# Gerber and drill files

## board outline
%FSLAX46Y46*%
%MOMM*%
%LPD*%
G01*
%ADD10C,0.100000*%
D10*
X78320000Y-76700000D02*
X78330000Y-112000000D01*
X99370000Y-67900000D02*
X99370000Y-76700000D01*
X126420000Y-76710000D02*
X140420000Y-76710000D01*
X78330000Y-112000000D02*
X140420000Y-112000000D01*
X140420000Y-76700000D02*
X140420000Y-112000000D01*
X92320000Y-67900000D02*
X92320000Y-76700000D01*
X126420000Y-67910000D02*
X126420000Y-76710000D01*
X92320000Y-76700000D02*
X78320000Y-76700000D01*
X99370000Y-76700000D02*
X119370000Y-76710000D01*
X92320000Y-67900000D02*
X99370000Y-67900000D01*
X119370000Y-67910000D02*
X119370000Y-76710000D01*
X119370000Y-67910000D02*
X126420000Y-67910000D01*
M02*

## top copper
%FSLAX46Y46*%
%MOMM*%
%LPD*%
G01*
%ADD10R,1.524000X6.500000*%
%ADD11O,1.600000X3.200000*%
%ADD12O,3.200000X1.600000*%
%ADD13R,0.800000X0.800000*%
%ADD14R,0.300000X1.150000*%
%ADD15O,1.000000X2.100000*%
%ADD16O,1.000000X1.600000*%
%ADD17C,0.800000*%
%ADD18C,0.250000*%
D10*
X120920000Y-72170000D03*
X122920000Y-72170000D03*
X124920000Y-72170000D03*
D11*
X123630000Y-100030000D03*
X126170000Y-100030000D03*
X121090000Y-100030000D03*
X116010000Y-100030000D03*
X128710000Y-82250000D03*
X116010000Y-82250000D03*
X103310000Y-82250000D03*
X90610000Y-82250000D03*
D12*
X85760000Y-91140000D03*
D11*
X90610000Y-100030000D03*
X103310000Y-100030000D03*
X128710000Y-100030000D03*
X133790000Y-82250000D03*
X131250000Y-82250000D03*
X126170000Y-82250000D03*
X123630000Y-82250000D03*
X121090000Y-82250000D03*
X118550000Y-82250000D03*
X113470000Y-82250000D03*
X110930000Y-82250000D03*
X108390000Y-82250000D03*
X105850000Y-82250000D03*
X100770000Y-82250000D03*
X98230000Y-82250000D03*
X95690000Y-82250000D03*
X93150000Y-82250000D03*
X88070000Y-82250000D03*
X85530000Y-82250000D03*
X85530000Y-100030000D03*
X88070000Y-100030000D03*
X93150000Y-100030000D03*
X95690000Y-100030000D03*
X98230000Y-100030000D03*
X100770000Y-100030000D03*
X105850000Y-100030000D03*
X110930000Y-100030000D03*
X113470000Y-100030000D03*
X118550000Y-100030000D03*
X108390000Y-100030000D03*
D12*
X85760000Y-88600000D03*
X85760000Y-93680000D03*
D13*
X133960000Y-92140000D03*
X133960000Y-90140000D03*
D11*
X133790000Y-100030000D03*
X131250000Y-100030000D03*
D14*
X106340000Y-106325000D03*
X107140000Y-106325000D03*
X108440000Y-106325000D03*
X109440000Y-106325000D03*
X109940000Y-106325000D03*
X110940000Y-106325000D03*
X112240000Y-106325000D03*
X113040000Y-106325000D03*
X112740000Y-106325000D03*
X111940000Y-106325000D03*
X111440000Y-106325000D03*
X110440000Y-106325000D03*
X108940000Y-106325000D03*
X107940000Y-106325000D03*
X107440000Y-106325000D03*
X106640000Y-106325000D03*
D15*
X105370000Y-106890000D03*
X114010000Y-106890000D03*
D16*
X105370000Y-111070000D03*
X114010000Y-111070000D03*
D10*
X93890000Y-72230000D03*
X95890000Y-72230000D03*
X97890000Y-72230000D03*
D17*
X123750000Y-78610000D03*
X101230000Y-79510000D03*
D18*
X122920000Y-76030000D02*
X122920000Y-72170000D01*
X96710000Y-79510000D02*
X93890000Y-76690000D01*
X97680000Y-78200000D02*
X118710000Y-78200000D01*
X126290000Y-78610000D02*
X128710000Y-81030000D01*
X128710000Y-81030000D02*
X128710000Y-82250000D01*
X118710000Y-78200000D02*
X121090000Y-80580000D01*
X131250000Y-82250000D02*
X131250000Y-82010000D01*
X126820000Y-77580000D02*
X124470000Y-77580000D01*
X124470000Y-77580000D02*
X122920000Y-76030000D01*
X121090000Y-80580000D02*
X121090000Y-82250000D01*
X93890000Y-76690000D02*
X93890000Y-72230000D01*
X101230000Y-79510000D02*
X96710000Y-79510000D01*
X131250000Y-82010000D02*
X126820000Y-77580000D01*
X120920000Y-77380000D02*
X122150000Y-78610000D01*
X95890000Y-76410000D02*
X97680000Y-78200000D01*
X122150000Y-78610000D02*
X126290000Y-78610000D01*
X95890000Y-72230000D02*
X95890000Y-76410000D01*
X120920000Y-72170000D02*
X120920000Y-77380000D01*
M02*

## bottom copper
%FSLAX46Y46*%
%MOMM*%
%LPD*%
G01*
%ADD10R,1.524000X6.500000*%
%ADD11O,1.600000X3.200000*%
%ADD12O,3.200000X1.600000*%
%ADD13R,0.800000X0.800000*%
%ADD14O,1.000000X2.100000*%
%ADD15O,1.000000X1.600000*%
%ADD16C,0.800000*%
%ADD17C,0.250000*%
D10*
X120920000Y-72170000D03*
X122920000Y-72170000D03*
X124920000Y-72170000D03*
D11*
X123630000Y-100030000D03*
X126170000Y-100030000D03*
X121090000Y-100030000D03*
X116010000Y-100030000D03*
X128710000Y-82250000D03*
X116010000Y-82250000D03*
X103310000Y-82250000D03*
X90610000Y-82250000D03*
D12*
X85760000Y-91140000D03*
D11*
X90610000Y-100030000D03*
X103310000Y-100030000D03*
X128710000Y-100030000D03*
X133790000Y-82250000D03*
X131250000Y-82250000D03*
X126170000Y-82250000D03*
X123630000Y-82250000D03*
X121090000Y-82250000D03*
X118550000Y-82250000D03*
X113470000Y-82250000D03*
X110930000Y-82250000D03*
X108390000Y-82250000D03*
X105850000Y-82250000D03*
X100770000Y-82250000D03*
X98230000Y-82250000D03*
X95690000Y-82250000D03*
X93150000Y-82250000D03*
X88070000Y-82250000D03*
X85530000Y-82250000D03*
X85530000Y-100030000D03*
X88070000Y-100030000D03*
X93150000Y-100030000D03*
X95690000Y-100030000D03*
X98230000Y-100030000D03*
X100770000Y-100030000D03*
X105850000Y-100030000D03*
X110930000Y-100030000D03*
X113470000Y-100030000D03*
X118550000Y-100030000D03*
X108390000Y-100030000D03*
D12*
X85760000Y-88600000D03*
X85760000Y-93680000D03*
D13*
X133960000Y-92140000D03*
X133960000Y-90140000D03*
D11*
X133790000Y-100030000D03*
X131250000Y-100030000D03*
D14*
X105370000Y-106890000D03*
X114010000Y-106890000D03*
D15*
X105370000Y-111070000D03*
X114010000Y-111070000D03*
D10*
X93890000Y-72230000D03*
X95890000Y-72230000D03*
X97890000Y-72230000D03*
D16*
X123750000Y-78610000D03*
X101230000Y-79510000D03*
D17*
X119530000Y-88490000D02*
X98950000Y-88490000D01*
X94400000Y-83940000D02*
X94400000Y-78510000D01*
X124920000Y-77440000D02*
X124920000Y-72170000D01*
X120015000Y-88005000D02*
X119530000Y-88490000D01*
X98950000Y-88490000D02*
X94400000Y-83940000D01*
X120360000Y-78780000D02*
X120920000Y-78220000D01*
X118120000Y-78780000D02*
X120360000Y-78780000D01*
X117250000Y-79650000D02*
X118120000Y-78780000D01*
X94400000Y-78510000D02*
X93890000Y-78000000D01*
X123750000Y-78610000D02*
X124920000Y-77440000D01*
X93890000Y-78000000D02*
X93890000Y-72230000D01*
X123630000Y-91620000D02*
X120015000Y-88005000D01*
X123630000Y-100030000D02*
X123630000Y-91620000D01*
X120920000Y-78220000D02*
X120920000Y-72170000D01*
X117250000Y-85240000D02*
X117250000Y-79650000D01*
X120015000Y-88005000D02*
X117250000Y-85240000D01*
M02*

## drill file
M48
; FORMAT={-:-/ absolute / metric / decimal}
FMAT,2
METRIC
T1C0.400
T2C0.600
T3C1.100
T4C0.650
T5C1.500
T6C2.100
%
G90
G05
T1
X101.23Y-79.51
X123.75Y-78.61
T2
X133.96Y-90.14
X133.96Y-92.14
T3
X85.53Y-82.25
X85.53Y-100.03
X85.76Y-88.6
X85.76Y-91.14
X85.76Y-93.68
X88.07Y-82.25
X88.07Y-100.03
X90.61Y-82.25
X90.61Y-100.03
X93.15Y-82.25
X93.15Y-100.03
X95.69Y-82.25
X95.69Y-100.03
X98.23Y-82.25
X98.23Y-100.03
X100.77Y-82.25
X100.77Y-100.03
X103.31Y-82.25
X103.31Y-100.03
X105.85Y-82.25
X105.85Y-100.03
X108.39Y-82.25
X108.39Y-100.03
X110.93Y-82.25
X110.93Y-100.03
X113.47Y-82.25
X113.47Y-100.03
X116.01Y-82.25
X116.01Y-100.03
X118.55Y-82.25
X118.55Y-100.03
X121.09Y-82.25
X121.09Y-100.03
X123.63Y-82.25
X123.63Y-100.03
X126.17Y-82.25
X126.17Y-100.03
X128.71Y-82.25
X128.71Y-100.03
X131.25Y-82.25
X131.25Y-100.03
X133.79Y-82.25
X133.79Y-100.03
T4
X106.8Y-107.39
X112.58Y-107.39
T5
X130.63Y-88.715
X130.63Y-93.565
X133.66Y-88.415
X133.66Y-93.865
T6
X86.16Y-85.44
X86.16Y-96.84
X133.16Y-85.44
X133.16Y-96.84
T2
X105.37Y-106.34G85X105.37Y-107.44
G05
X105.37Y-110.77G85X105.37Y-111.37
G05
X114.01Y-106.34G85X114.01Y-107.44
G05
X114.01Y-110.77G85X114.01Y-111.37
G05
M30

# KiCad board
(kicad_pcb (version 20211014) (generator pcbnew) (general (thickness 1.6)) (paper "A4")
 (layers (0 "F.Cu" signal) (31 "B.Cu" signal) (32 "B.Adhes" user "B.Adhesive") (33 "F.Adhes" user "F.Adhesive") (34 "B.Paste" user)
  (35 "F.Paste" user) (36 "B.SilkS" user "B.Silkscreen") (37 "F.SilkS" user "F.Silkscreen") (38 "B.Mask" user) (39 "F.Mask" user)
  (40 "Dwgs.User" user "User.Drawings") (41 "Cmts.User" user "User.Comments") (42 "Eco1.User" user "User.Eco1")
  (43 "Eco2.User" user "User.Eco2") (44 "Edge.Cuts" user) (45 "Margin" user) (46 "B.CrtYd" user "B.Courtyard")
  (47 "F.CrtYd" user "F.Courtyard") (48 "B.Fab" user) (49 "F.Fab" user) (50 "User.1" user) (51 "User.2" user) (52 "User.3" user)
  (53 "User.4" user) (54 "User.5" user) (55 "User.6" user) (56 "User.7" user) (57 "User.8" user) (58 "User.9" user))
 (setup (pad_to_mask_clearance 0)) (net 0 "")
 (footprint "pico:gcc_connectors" (layer "F.Cu") (at 123.27 72.17)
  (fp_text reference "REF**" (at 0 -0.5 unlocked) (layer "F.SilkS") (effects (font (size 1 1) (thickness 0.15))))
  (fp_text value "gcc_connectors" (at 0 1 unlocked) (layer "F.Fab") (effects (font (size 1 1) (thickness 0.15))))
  (pad "1" smd rect (at -2.35 0) (size 1.524 6.5) (layers "F.Cu" "F.Paste" "F.Mask"))
  (pad "2" smd rect (at -0.35 0) (size 1.524 6.5) (layers "F.Cu" "F.Paste" "F.Mask"))
  (pad "3" smd rect (at 1.65 0) (size 1.524 6.5) (layers "F.Cu" "F.Paste" "F.Mask"))
  (pad "4" smd rect (at -2.35 0) (size 1.524 6.5) (layers "B.Cu" "B.Paste" "B.Mask"))
  (pad "5" smd rect (at -0.35 0) (size 1.524 6.5) (layers "B.Cu" "B.Paste" "B.Mask"))
  (pad "6" smd rect (at 1.65 0) (size 1.524 6.5) (layers "B.Cu" "B.Paste" "B.Mask")))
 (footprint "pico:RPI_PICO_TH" (layer "F.Cu") (at 109.66 91.14 -90)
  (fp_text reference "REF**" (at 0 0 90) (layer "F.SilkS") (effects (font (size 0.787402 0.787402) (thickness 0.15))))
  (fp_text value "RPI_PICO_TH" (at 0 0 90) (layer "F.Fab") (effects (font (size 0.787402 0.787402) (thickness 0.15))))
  (pad "" np_thru_hole circle locked (at -5.7 23.5 270) (size 2.1 2.1) (drill 2.1) (layers *.Cu *.Mask))
  (pad "" np_thru_hole circle locked (at -2.425 -20.97 270) (size 1.5 1.5) (drill 1.5) (layers *.Cu *.Mask))
  (pad "" np_thru_hole circle locked (at -5.7 -23.5 270) (size 2.1 2.1) (drill 2.1) (layers *.Cu *.Mask))
  (pad "" np_thru_hole circle locked (at 2.425 -20.97 270) (size 1.5 1.5) (drill 1.5) (layers *.Cu *.Mask))
  (pad "" np_thru_hole circle locked (at 2.725 -24 270) (size 1.5 1.5) (drill 1.5) (layers *.Cu *.Mask))
  (pad "" np_thru_hole circle locked (at 5.7 23.5 270) (size 2.1 2.1) (drill 2.1) (layers *.Cu *.Mask))
  (pad "" np_thru_hole circle locked (at 5.7 -23.5 270) (size 2.1 2.1) (drill 2.1) (layers *.Cu *.Mask))
  (pad "" np_thru_hole circle locked (at -2.725 -24 270) (size 1.5 1.5) (drill 1.5) (layers *.Cu *.Mask))
  (pad "3V3" thru_hole oval locked (at 8.89 -13.97 270) (size 3.2 1.6) (drill 1.1) (layers *.Cu *.Mask))
  (pad "3V3_EN" thru_hole oval locked (at 8.89 -16.51 270) (size 3.2 1.6) (drill 1.1) (layers *.Cu *.Mask))
  (pad "ADC_VREF" thru_hole oval locked (at 8.89 -11.43 270) (size 3.2 1.6) (drill 1.1) (layers *.Cu *.Mask))
  (pad "AGND" thru_hole oval locked (at 8.89 -6.35 270) (size 3.2 1.6) (drill 1.1) (layers *.Cu *.Mask))
  (pad "GND@1" thru_hole oval locked (at -8.89 -19.05 270) (size 3.2 1.6) (drill 1.1) (layers *.Cu *.Mask))
  (pad "GND@2" thru_hole oval locked (at -8.89 -6.35 270) (size 3.2 1.6) (drill 1.1) (layers *.Cu *.Mask))
  (pad "GND@3" thru_hole oval locked (at -8.89 6.35 270) (size 3.2 1.6) (drill 1.1) (layers *.Cu *.Mask))
  (pad "GND@4" thru_hole oval locked (at -8.89 19.05 270) (size 3.2 1.6) (drill 1.1) (layers *.Cu *.Mask))
  (pad "GND@5" thru_hole oval locked (at 0 23.9 270) (size 1.6 3.2) (drill 1.1) (layers *.Cu *.Mask))
  (pad "GND@6" thru_hole oval locked (at 8.89 19.05 270) (size 3.2 1.6) (drill 1.1) (layers *.Cu *.Mask))
  (pad "GND@7" thru_hole oval locked (at 8.89 6.35 270) (size 3.2 1.6) (drill 1.1) (layers *.Cu *.Mask))
  (pad "GND@8" thru_hole oval locked (at 8.89 -19.05 270) (size 3.2 1.6) (drill 1.1) (layers *.Cu *.Mask))
  (pad "GP0" thru_hole oval locked (at -8.89 -24.13 270) (size 3.2 1.6) (drill 1.1) (layers *.Cu *.Mask))
  (pad "GP1" thru_hole oval locked (at -8.89 -21.59 270) (size 3.2 1.6) (drill 1.1) (layers *.Cu *.Mask))
  (pad "GP2" thru_hole oval locked (at -8.89 -16.51 270) (size 3.2 1.6) (drill 1.1) (layers *.Cu *.Mask))
  (pad "GP3" thru_hole oval locked (at -8.89 -13.97 270) (size 3.2 1.6) (drill 1.1) (layers *.Cu *.Mask))
  (pad "GP4" thru_hole oval locked (at -8.89 -11.43 270) (size 3.2 1.6) (drill 1.1) (layers *.Cu *.Mask))
  (pad "GP5" thru_hole oval locked (at -8.89 -8.89 270) (size 3.2 1.6) (drill 1.1) (layers *.Cu *.Mask))
  (pad "GP6" thru_hole oval locked (at -8.89 -3.81 270) (size 3.2 1.6) (drill 1.1) (layers *.Cu *.Mask))
  (pad "GP7" thru_hole oval locked (at -8.89 -1.27 270) (size 3.2 1.6) (drill 1.1) (layers *.Cu *.Mask))
  (pad "GP8" thru_hole oval locked (at -8.89 1.27 270) (size 3.2 1.6) (drill 1.1) (layers *.Cu *.Mask))
  (pad "GP9" thru_hole oval locked (at -8.89 3.81 270) (size 3.2 1.6) (drill 1.1) (layers *.Cu *.Mask))
  (pad "GP10" thru_hole oval locked (at -8.89 8.89 270) (size 3.2 1.6) (drill 1.1) (layers *.Cu *.Mask))
  (pad "GP11" thru_hole oval locked (at -8.89 11.43 270) (size 3.2 1.6) (drill 1.1) (layers *.Cu *.Mask))
  (pad "GP12" thru_hole oval locked (at -8.89 13.97 270) (size 3.2 1.6) (drill 1.1) (layers *.Cu *.Mask))
  (pad "GP13" thru_hole oval locked (at -8.89 16.51 270) (size 3.2 1.6) (drill 1.1) (layers *.Cu *.Mask))
  (pad "GP14" thru_hole oval locked (at -8.89 21.59 270) (size 3.2 1.6) (drill 1.1) (layers *.Cu *.Mask))
  (pad "GP15" thru_hole oval locked (at -8.89 24.13 270) (size 3.2 1.6) (drill 1.1) (layers *.Cu *.Mask))
  (pad "GP16" thru_hole oval locked (at 8.89 24.13 270) (size 3.2 1.6) (drill 1.1) (layers *.Cu *.Mask))
  (pad "GP17" thru_hole oval locked (at 8.89 21.59 270) (size 3.2 1.6) (drill 1.1) (layers *.Cu *.Mask))
  (pad "GP18" thru_hole oval locked (at 8.89 16.51 270) (size 3.2 1.6) (drill 1.1) (layers *.Cu *.Mask))
  (pad "GP19" thru_hole oval locked (at 8.89 13.97 270) (size 3.2 1.6) (drill 1.1) (layers *.Cu *.Mask))
  (pad "GP20" thru_hole oval locked (at 8.89 11.43 270) (size 3.2 1.6) (drill 1.1) (layers *.Cu *.Mask))
  (pad "GP21" thru_hole oval locked (at 8.89 8.89 270) (size 3.2 1.6) (drill 1.1) (layers *.Cu *.Mask))
  (pad "GP22" thru_hole oval locked (at 8.89 3.81 270) (size 3.2 1.6) (drill 1.1) (layers *.Cu *.Mask))
  (pad "GP26_A0" thru_hole oval locked (at 8.89 -1.27 270) (size 3.2 1.6) (drill 1.1) (layers *.Cu *.Mask))
  (pad "GP27_A1" thru_hole oval locked (at 8.89 -3.81 270) (size 3.2 1.6) (drill 1.1) (layers *.Cu *.Mask))
  (pad "GP28_A2" thru_hole oval locked (at 8.89 -8.89 270) (size 3.2 1.6) (drill 1.1) (layers *.Cu *.Mask))
  (pad "RUN" thru_hole oval locked (at 8.89 1.27 270) (size 3.2 1.6) (drill 1.1) (layers *.Cu *.Mask))
  (pad "SWCLK" thru_hole oval locked (at -2.54 23.9 270) (size 1.6 3.2) (drill 1.1) (layers *.Cu *.Mask))
  (pad "SWDIO" thru_hole oval locked (at 2.54 23.9 270) (size 1.6 3.2) (drill 1.1) (layers *.Cu *.Mask))
  (pad "TP2" thru_hole rect locked (at 1 -24.3 270) (size 0.8 0.8) (drill 0.6) (layers *.Cu *.Mask))
  (pad "TP3" thru_hole rect locked (at -1 -24.3 270) (size 0.8 0.8) (drill 0.6) (layers *.Cu *.Mask))
  (pad "VBUS" thru_hole oval locked (at 8.89 -24.13 270) (size 3.2 1.6) (drill 1.1) (layers *.Cu *.Mask))
  (pad "VSYS" thru_hole oval locked (at 8.89 -21.59 270) (size 3.2 1.6) (drill 1.1) (layers *.Cu *.Mask)))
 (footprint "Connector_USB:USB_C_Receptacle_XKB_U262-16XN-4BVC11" (layer "F.Cu") (at 109.69 109.995)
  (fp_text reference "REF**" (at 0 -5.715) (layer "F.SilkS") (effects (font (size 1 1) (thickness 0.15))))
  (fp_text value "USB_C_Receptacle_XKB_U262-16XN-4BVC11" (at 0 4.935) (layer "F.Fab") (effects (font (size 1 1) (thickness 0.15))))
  (pad "" np_thru_hole circle (at -2.89 -2.605) (size 0.65 0.65) (drill 0.65) (layers *.Cu *.Mask))
  (pad "" np_thru_hole circle (at 2.89 -2.605) (size 0.65 0.65) (drill 0.65) (layers *.Cu *.Mask))
  (pad "A1" smd rect (at -3.35 -3.67) (size 0.3 1.15) (layers "F.Cu" "F.Paste" "F.Mask"))
  (pad "A4" smd rect (at -2.55 -3.67) (size 0.3 1.15) (layers "F.Cu" "F.Paste" "F.Mask"))
  (pad "A5" smd rect (at -1.25 -3.67) (size 0.3 1.15) (layers "F.Cu" "F.Paste" "F.Mask"))
  (pad "A6" smd rect (at -0.25 -3.67) (size 0.3 1.15) (layers "F.Cu" "F.Paste" "F.Mask"))
  (pad "A7" smd rect (at 0.25 -3.67) (size 0.3 1.15) (layers "F.Cu" "F.Paste" "F.Mask"))
  (pad "A8" smd rect (at 1.25 -3.67) (size 0.3 1.15) (layers "F.Cu" "F.Paste" "F.Mask"))
  (pad "A9" smd rect (at 2.55 -3.67) (size 0.3 1.15) (layers "F.Cu" "F.Paste" "F.Mask"))
  (pad "A12" smd rect (at 3.35 -3.67) (size 0.3 1.15) (layers "F.Cu" "F.Paste" "F.Mask"))
  (pad "B1" smd rect (at 3.05 -3.67) (size 0.3 1.15) (layers "F.Cu" "F.Paste" "F.Mask"))
  (pad "B4" smd rect (at 2.25 -3.67) (size 0.3 1.15) (layers "F.Cu" "F.Paste" "F.Mask"))
  (pad "B5" smd rect (at 1.75 -3.67) (size 0.3 1.15) (layers "F.Cu" "F.Paste" "F.Mask"))
  (pad "B6" smd rect (at 0.75 -3.67) (size 0.3 1.15) (layers "F.Cu" "F.Paste" "F.Mask"))
  (pad "B7" smd rect (at -0.75 -3.67) (size 0.3 1.15) (layers "F.Cu" "F.Paste" "F.Mask"))
  (pad "B8" smd rect (at -1.75 -3.67) (size 0.3 1.15) (layers "F.Cu" "F.Paste" "F.Mask"))
  (pad "B9" smd rect (at -2.25 -3.67) (size 0.3 1.15) (layers "F.Cu" "F.Paste" "F.Mask"))
  (pad "B12" smd rect (at -3.05 -3.67) (size 0.3 1.15) (layers "F.Cu" "F.Paste" "F.Mask"))
  (pad "S1" thru_hole oval (at -4.32 -3.105) (size 1 2.1) (drill oval 0.6 1.7) (layers *.Cu *.Mask))
  (pad "S1" thru_hole oval (at 4.32 -3.105) (size 1 2.1) (drill oval 0.6 1.7) (layers *.Cu *.Mask))
  (pad "S1" thru_hole oval (at -4.32 1.075) (size 1 1.6) (drill oval 0.6 1.2) (layers *.Cu *.Mask))
  (pad "S1" thru_hole oval (at 4.32 1.075) (size 1 1.6) (drill oval 0.6 1.2) (layers *.Cu *.Mask)))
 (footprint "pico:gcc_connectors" (layer "F.Cu") (at 96.24 72.23)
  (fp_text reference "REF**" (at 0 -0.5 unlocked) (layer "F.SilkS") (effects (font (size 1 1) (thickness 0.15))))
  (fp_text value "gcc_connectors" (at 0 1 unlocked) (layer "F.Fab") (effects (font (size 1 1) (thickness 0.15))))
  (pad "1" smd rect (at -2.35 0) (size 1.524 6.5) (layers "F.Cu" "F.Paste" "F.Mask"))
  (pad "2" smd rect (at -0.35 0) (size 1.524 6.5) (layers "F.Cu" "F.Paste" "F.Mask"))
  (pad "3" smd rect (at 1.65 0) (size 1.524 6.5) (layers "F.Cu" "F.Paste" "F.Mask"))
  (pad "4" smd rect (at -2.35 0) (size 1.524 6.5) (layers "B.Cu" "B.Paste" "B.Mask"))
  (pad "5" smd rect (at -0.35 0) (size 1.524 6.5) (layers "B.Cu" "B.Paste" "B.Mask"))
  (pad "6" smd rect (at 1.65 0) (size 1.524 6.5) (layers "B.Cu" "B.Paste" "B.Mask")))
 (gr_line (start 78.32 76.7) (end 78.33 112) (layer "Edge.Cuts") (width 0.1))
 (gr_line (start 99.37 67.9) (end 99.37 76.7) (layer "Edge.Cuts") (width 0.1))
 (gr_line (start 126.42 76.71) (end 140.42 76.71) (layer "Edge.Cuts") (width 0.1))
 (gr_line (start 78.33 112) (end 140.42 112) (layer "Edge.Cuts") (width 0.1))
 (gr_line (start 140.42 76.7) (end 140.42 112) (layer "Edge.Cuts") (width 0.1))
 (gr_line (start 92.32 67.9) (end 92.32 76.7) (layer "Edge.Cuts") (width 0.1))
 (gr_line (start 126.42 67.91) (end 126.42 76.71) (layer "Edge.Cuts") (width 0.1))
 (gr_line (start 92.32 76.7) (end 78.32 76.7) (layer "Edge.Cuts") (width 0.1))
 (gr_line (start 99.37 76.7) (end 119.37 76.71) (layer "Edge.Cuts") (width 0.1))
 (gr_line (start 92.32 67.9) (end 99.37 67.9) (layer "Edge.Cuts") (width 0.1))
 (gr_line (start 119.37 67.91) (end 119.37 76.71) (layer "Edge.Cuts") (width 0.1))
 (gr_line (start 119.37 67.91) (end 126.42 67.91) (layer "Edge.Cuts") (width 0.1))
 (segment (start 122.92 76.03) (end 122.92 72.17) (width 0.25) (layer "F.Cu") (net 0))
 (segment (start 96.71 79.51) (end 93.89 76.69) (width 0.25) (layer "F.Cu") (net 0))
 (segment (start 97.68 78.2) (end 118.71 78.2) (width 0.25) (layer "F.Cu") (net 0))
 (segment (start 126.29 78.61) (end 128.71 81.03) (width 0.25) (layer "F.Cu") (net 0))
 (segment (start 128.71 81.03) (end 128.71 82.25) (width 0.25) (layer "F.Cu") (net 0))
 (segment (start 118.71 78.2) (end 121.09 80.58) (width 0.25) (layer "F.Cu") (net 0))
 (segment (start 131.25 82.25) (end 131.25 82.01) (width 0.25) (layer "F.Cu") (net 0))
 (segment (start 126.82 77.58) (end 124.47 77.58) (width 0.25) (layer "F.Cu") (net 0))
 (segment (start 124.47 77.58) (end 122.92 76.03) (width 0.25) (layer "F.Cu") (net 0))
 (segment (start 121.09 80.58) (end 121.09 82.25) (width 0.25) (layer "F.Cu") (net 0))
 (segment (start 93.89 76.69) (end 93.89 72.23) (width 0.25) (layer "F.Cu") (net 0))
 (segment (start 101.23 79.51) (end 96.71 79.51) (width 0.25) (layer "F.Cu") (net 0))
 (segment (start 131.25 82.01) (end 126.82 77.58) (width 0.25) (layer "F.Cu") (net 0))
 (segment (start 120.92 77.38) (end 122.15 78.61) (width 0.25) (layer "F.Cu") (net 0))
 (segment (start 95.89 76.41) (end 97.68 78.2) (width 0.25) (layer "F.Cu") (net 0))
 (segment (start 122.15 78.61) (end 126.29 78.61) (width 0.25) (layer "F.Cu") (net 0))
 (segment (start 95.89 72.23) (end 95.89 76.41) (width 0.25) (layer "F.Cu") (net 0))
 (segment (start 120.92 72.17) (end 120.92 77.38) (width 0.25) (layer "F.Cu") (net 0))
 (via (at 123.75 78.61) (size 0.8) (drill 0.4) (layers "F.Cu" "B.Cu") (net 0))
 (via (at 101.23 79.51) (size 0.8) (drill 0.4) (layers "F.Cu" "B.Cu") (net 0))
 (segment (start 119.53 88.49) (end 98.95 88.49) (width 0.25) (layer "B.Cu") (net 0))
 (segment (start 94.4 83.94) (end 94.4 78.51) (width 0.25) (layer "B.Cu") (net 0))
 (segment (start 124.92 77.44) (end 124.92 72.17) (width 0.25) (layer "B.Cu") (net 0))
 (segment (start 120.015 88.005) (end 119.53 88.49) (width 0.25) (layer "B.Cu") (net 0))
 (segment (start 98.95 88.49) (end 94.4 83.94) (width 0.25) (layer "B.Cu") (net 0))
 (segment (start 120.36 78.78) (end 120.92 78.22) (width 0.25) (layer "B.Cu") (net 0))
 (segment (start 118.12 78.78) (end 120.36 78.78) (width 0.25) (layer "B.Cu") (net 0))
 (segment (start 117.25 79.65) (end 118.12 78.78) (width 0.25) (layer "B.Cu") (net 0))
 (segment (start 94.4 78.51) (end 93.89 78) (width 0.25) (layer "B.Cu") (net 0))
 (segment (start 123.75 78.61) (end 124.92 77.44) (width 0.25) (layer "B.Cu") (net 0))
 (segment (start 93.89 78) (end 93.89 72.23) (width 0.25) (layer "B.Cu") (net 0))
 (segment (start 123.63 91.62) (end 120.015 88.005) (width 0.25) (layer "B.Cu") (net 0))
 (segment (start 123.63 100.03) (end 123.63 91.62) (width 0.25) (layer "B.Cu") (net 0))
 (segment (start 120.92 78.22) (end 120.92 72.17) (width 0.25) (layer "B.Cu") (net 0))
 (segment (start 117.25 85.24) (end 117.25 79.65) (width 0.25) (layer "B.Cu") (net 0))
 (segment (start 120.015 88.005) (end 117.25 85.24) (width 0.25) (layer "B.Cu") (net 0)))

